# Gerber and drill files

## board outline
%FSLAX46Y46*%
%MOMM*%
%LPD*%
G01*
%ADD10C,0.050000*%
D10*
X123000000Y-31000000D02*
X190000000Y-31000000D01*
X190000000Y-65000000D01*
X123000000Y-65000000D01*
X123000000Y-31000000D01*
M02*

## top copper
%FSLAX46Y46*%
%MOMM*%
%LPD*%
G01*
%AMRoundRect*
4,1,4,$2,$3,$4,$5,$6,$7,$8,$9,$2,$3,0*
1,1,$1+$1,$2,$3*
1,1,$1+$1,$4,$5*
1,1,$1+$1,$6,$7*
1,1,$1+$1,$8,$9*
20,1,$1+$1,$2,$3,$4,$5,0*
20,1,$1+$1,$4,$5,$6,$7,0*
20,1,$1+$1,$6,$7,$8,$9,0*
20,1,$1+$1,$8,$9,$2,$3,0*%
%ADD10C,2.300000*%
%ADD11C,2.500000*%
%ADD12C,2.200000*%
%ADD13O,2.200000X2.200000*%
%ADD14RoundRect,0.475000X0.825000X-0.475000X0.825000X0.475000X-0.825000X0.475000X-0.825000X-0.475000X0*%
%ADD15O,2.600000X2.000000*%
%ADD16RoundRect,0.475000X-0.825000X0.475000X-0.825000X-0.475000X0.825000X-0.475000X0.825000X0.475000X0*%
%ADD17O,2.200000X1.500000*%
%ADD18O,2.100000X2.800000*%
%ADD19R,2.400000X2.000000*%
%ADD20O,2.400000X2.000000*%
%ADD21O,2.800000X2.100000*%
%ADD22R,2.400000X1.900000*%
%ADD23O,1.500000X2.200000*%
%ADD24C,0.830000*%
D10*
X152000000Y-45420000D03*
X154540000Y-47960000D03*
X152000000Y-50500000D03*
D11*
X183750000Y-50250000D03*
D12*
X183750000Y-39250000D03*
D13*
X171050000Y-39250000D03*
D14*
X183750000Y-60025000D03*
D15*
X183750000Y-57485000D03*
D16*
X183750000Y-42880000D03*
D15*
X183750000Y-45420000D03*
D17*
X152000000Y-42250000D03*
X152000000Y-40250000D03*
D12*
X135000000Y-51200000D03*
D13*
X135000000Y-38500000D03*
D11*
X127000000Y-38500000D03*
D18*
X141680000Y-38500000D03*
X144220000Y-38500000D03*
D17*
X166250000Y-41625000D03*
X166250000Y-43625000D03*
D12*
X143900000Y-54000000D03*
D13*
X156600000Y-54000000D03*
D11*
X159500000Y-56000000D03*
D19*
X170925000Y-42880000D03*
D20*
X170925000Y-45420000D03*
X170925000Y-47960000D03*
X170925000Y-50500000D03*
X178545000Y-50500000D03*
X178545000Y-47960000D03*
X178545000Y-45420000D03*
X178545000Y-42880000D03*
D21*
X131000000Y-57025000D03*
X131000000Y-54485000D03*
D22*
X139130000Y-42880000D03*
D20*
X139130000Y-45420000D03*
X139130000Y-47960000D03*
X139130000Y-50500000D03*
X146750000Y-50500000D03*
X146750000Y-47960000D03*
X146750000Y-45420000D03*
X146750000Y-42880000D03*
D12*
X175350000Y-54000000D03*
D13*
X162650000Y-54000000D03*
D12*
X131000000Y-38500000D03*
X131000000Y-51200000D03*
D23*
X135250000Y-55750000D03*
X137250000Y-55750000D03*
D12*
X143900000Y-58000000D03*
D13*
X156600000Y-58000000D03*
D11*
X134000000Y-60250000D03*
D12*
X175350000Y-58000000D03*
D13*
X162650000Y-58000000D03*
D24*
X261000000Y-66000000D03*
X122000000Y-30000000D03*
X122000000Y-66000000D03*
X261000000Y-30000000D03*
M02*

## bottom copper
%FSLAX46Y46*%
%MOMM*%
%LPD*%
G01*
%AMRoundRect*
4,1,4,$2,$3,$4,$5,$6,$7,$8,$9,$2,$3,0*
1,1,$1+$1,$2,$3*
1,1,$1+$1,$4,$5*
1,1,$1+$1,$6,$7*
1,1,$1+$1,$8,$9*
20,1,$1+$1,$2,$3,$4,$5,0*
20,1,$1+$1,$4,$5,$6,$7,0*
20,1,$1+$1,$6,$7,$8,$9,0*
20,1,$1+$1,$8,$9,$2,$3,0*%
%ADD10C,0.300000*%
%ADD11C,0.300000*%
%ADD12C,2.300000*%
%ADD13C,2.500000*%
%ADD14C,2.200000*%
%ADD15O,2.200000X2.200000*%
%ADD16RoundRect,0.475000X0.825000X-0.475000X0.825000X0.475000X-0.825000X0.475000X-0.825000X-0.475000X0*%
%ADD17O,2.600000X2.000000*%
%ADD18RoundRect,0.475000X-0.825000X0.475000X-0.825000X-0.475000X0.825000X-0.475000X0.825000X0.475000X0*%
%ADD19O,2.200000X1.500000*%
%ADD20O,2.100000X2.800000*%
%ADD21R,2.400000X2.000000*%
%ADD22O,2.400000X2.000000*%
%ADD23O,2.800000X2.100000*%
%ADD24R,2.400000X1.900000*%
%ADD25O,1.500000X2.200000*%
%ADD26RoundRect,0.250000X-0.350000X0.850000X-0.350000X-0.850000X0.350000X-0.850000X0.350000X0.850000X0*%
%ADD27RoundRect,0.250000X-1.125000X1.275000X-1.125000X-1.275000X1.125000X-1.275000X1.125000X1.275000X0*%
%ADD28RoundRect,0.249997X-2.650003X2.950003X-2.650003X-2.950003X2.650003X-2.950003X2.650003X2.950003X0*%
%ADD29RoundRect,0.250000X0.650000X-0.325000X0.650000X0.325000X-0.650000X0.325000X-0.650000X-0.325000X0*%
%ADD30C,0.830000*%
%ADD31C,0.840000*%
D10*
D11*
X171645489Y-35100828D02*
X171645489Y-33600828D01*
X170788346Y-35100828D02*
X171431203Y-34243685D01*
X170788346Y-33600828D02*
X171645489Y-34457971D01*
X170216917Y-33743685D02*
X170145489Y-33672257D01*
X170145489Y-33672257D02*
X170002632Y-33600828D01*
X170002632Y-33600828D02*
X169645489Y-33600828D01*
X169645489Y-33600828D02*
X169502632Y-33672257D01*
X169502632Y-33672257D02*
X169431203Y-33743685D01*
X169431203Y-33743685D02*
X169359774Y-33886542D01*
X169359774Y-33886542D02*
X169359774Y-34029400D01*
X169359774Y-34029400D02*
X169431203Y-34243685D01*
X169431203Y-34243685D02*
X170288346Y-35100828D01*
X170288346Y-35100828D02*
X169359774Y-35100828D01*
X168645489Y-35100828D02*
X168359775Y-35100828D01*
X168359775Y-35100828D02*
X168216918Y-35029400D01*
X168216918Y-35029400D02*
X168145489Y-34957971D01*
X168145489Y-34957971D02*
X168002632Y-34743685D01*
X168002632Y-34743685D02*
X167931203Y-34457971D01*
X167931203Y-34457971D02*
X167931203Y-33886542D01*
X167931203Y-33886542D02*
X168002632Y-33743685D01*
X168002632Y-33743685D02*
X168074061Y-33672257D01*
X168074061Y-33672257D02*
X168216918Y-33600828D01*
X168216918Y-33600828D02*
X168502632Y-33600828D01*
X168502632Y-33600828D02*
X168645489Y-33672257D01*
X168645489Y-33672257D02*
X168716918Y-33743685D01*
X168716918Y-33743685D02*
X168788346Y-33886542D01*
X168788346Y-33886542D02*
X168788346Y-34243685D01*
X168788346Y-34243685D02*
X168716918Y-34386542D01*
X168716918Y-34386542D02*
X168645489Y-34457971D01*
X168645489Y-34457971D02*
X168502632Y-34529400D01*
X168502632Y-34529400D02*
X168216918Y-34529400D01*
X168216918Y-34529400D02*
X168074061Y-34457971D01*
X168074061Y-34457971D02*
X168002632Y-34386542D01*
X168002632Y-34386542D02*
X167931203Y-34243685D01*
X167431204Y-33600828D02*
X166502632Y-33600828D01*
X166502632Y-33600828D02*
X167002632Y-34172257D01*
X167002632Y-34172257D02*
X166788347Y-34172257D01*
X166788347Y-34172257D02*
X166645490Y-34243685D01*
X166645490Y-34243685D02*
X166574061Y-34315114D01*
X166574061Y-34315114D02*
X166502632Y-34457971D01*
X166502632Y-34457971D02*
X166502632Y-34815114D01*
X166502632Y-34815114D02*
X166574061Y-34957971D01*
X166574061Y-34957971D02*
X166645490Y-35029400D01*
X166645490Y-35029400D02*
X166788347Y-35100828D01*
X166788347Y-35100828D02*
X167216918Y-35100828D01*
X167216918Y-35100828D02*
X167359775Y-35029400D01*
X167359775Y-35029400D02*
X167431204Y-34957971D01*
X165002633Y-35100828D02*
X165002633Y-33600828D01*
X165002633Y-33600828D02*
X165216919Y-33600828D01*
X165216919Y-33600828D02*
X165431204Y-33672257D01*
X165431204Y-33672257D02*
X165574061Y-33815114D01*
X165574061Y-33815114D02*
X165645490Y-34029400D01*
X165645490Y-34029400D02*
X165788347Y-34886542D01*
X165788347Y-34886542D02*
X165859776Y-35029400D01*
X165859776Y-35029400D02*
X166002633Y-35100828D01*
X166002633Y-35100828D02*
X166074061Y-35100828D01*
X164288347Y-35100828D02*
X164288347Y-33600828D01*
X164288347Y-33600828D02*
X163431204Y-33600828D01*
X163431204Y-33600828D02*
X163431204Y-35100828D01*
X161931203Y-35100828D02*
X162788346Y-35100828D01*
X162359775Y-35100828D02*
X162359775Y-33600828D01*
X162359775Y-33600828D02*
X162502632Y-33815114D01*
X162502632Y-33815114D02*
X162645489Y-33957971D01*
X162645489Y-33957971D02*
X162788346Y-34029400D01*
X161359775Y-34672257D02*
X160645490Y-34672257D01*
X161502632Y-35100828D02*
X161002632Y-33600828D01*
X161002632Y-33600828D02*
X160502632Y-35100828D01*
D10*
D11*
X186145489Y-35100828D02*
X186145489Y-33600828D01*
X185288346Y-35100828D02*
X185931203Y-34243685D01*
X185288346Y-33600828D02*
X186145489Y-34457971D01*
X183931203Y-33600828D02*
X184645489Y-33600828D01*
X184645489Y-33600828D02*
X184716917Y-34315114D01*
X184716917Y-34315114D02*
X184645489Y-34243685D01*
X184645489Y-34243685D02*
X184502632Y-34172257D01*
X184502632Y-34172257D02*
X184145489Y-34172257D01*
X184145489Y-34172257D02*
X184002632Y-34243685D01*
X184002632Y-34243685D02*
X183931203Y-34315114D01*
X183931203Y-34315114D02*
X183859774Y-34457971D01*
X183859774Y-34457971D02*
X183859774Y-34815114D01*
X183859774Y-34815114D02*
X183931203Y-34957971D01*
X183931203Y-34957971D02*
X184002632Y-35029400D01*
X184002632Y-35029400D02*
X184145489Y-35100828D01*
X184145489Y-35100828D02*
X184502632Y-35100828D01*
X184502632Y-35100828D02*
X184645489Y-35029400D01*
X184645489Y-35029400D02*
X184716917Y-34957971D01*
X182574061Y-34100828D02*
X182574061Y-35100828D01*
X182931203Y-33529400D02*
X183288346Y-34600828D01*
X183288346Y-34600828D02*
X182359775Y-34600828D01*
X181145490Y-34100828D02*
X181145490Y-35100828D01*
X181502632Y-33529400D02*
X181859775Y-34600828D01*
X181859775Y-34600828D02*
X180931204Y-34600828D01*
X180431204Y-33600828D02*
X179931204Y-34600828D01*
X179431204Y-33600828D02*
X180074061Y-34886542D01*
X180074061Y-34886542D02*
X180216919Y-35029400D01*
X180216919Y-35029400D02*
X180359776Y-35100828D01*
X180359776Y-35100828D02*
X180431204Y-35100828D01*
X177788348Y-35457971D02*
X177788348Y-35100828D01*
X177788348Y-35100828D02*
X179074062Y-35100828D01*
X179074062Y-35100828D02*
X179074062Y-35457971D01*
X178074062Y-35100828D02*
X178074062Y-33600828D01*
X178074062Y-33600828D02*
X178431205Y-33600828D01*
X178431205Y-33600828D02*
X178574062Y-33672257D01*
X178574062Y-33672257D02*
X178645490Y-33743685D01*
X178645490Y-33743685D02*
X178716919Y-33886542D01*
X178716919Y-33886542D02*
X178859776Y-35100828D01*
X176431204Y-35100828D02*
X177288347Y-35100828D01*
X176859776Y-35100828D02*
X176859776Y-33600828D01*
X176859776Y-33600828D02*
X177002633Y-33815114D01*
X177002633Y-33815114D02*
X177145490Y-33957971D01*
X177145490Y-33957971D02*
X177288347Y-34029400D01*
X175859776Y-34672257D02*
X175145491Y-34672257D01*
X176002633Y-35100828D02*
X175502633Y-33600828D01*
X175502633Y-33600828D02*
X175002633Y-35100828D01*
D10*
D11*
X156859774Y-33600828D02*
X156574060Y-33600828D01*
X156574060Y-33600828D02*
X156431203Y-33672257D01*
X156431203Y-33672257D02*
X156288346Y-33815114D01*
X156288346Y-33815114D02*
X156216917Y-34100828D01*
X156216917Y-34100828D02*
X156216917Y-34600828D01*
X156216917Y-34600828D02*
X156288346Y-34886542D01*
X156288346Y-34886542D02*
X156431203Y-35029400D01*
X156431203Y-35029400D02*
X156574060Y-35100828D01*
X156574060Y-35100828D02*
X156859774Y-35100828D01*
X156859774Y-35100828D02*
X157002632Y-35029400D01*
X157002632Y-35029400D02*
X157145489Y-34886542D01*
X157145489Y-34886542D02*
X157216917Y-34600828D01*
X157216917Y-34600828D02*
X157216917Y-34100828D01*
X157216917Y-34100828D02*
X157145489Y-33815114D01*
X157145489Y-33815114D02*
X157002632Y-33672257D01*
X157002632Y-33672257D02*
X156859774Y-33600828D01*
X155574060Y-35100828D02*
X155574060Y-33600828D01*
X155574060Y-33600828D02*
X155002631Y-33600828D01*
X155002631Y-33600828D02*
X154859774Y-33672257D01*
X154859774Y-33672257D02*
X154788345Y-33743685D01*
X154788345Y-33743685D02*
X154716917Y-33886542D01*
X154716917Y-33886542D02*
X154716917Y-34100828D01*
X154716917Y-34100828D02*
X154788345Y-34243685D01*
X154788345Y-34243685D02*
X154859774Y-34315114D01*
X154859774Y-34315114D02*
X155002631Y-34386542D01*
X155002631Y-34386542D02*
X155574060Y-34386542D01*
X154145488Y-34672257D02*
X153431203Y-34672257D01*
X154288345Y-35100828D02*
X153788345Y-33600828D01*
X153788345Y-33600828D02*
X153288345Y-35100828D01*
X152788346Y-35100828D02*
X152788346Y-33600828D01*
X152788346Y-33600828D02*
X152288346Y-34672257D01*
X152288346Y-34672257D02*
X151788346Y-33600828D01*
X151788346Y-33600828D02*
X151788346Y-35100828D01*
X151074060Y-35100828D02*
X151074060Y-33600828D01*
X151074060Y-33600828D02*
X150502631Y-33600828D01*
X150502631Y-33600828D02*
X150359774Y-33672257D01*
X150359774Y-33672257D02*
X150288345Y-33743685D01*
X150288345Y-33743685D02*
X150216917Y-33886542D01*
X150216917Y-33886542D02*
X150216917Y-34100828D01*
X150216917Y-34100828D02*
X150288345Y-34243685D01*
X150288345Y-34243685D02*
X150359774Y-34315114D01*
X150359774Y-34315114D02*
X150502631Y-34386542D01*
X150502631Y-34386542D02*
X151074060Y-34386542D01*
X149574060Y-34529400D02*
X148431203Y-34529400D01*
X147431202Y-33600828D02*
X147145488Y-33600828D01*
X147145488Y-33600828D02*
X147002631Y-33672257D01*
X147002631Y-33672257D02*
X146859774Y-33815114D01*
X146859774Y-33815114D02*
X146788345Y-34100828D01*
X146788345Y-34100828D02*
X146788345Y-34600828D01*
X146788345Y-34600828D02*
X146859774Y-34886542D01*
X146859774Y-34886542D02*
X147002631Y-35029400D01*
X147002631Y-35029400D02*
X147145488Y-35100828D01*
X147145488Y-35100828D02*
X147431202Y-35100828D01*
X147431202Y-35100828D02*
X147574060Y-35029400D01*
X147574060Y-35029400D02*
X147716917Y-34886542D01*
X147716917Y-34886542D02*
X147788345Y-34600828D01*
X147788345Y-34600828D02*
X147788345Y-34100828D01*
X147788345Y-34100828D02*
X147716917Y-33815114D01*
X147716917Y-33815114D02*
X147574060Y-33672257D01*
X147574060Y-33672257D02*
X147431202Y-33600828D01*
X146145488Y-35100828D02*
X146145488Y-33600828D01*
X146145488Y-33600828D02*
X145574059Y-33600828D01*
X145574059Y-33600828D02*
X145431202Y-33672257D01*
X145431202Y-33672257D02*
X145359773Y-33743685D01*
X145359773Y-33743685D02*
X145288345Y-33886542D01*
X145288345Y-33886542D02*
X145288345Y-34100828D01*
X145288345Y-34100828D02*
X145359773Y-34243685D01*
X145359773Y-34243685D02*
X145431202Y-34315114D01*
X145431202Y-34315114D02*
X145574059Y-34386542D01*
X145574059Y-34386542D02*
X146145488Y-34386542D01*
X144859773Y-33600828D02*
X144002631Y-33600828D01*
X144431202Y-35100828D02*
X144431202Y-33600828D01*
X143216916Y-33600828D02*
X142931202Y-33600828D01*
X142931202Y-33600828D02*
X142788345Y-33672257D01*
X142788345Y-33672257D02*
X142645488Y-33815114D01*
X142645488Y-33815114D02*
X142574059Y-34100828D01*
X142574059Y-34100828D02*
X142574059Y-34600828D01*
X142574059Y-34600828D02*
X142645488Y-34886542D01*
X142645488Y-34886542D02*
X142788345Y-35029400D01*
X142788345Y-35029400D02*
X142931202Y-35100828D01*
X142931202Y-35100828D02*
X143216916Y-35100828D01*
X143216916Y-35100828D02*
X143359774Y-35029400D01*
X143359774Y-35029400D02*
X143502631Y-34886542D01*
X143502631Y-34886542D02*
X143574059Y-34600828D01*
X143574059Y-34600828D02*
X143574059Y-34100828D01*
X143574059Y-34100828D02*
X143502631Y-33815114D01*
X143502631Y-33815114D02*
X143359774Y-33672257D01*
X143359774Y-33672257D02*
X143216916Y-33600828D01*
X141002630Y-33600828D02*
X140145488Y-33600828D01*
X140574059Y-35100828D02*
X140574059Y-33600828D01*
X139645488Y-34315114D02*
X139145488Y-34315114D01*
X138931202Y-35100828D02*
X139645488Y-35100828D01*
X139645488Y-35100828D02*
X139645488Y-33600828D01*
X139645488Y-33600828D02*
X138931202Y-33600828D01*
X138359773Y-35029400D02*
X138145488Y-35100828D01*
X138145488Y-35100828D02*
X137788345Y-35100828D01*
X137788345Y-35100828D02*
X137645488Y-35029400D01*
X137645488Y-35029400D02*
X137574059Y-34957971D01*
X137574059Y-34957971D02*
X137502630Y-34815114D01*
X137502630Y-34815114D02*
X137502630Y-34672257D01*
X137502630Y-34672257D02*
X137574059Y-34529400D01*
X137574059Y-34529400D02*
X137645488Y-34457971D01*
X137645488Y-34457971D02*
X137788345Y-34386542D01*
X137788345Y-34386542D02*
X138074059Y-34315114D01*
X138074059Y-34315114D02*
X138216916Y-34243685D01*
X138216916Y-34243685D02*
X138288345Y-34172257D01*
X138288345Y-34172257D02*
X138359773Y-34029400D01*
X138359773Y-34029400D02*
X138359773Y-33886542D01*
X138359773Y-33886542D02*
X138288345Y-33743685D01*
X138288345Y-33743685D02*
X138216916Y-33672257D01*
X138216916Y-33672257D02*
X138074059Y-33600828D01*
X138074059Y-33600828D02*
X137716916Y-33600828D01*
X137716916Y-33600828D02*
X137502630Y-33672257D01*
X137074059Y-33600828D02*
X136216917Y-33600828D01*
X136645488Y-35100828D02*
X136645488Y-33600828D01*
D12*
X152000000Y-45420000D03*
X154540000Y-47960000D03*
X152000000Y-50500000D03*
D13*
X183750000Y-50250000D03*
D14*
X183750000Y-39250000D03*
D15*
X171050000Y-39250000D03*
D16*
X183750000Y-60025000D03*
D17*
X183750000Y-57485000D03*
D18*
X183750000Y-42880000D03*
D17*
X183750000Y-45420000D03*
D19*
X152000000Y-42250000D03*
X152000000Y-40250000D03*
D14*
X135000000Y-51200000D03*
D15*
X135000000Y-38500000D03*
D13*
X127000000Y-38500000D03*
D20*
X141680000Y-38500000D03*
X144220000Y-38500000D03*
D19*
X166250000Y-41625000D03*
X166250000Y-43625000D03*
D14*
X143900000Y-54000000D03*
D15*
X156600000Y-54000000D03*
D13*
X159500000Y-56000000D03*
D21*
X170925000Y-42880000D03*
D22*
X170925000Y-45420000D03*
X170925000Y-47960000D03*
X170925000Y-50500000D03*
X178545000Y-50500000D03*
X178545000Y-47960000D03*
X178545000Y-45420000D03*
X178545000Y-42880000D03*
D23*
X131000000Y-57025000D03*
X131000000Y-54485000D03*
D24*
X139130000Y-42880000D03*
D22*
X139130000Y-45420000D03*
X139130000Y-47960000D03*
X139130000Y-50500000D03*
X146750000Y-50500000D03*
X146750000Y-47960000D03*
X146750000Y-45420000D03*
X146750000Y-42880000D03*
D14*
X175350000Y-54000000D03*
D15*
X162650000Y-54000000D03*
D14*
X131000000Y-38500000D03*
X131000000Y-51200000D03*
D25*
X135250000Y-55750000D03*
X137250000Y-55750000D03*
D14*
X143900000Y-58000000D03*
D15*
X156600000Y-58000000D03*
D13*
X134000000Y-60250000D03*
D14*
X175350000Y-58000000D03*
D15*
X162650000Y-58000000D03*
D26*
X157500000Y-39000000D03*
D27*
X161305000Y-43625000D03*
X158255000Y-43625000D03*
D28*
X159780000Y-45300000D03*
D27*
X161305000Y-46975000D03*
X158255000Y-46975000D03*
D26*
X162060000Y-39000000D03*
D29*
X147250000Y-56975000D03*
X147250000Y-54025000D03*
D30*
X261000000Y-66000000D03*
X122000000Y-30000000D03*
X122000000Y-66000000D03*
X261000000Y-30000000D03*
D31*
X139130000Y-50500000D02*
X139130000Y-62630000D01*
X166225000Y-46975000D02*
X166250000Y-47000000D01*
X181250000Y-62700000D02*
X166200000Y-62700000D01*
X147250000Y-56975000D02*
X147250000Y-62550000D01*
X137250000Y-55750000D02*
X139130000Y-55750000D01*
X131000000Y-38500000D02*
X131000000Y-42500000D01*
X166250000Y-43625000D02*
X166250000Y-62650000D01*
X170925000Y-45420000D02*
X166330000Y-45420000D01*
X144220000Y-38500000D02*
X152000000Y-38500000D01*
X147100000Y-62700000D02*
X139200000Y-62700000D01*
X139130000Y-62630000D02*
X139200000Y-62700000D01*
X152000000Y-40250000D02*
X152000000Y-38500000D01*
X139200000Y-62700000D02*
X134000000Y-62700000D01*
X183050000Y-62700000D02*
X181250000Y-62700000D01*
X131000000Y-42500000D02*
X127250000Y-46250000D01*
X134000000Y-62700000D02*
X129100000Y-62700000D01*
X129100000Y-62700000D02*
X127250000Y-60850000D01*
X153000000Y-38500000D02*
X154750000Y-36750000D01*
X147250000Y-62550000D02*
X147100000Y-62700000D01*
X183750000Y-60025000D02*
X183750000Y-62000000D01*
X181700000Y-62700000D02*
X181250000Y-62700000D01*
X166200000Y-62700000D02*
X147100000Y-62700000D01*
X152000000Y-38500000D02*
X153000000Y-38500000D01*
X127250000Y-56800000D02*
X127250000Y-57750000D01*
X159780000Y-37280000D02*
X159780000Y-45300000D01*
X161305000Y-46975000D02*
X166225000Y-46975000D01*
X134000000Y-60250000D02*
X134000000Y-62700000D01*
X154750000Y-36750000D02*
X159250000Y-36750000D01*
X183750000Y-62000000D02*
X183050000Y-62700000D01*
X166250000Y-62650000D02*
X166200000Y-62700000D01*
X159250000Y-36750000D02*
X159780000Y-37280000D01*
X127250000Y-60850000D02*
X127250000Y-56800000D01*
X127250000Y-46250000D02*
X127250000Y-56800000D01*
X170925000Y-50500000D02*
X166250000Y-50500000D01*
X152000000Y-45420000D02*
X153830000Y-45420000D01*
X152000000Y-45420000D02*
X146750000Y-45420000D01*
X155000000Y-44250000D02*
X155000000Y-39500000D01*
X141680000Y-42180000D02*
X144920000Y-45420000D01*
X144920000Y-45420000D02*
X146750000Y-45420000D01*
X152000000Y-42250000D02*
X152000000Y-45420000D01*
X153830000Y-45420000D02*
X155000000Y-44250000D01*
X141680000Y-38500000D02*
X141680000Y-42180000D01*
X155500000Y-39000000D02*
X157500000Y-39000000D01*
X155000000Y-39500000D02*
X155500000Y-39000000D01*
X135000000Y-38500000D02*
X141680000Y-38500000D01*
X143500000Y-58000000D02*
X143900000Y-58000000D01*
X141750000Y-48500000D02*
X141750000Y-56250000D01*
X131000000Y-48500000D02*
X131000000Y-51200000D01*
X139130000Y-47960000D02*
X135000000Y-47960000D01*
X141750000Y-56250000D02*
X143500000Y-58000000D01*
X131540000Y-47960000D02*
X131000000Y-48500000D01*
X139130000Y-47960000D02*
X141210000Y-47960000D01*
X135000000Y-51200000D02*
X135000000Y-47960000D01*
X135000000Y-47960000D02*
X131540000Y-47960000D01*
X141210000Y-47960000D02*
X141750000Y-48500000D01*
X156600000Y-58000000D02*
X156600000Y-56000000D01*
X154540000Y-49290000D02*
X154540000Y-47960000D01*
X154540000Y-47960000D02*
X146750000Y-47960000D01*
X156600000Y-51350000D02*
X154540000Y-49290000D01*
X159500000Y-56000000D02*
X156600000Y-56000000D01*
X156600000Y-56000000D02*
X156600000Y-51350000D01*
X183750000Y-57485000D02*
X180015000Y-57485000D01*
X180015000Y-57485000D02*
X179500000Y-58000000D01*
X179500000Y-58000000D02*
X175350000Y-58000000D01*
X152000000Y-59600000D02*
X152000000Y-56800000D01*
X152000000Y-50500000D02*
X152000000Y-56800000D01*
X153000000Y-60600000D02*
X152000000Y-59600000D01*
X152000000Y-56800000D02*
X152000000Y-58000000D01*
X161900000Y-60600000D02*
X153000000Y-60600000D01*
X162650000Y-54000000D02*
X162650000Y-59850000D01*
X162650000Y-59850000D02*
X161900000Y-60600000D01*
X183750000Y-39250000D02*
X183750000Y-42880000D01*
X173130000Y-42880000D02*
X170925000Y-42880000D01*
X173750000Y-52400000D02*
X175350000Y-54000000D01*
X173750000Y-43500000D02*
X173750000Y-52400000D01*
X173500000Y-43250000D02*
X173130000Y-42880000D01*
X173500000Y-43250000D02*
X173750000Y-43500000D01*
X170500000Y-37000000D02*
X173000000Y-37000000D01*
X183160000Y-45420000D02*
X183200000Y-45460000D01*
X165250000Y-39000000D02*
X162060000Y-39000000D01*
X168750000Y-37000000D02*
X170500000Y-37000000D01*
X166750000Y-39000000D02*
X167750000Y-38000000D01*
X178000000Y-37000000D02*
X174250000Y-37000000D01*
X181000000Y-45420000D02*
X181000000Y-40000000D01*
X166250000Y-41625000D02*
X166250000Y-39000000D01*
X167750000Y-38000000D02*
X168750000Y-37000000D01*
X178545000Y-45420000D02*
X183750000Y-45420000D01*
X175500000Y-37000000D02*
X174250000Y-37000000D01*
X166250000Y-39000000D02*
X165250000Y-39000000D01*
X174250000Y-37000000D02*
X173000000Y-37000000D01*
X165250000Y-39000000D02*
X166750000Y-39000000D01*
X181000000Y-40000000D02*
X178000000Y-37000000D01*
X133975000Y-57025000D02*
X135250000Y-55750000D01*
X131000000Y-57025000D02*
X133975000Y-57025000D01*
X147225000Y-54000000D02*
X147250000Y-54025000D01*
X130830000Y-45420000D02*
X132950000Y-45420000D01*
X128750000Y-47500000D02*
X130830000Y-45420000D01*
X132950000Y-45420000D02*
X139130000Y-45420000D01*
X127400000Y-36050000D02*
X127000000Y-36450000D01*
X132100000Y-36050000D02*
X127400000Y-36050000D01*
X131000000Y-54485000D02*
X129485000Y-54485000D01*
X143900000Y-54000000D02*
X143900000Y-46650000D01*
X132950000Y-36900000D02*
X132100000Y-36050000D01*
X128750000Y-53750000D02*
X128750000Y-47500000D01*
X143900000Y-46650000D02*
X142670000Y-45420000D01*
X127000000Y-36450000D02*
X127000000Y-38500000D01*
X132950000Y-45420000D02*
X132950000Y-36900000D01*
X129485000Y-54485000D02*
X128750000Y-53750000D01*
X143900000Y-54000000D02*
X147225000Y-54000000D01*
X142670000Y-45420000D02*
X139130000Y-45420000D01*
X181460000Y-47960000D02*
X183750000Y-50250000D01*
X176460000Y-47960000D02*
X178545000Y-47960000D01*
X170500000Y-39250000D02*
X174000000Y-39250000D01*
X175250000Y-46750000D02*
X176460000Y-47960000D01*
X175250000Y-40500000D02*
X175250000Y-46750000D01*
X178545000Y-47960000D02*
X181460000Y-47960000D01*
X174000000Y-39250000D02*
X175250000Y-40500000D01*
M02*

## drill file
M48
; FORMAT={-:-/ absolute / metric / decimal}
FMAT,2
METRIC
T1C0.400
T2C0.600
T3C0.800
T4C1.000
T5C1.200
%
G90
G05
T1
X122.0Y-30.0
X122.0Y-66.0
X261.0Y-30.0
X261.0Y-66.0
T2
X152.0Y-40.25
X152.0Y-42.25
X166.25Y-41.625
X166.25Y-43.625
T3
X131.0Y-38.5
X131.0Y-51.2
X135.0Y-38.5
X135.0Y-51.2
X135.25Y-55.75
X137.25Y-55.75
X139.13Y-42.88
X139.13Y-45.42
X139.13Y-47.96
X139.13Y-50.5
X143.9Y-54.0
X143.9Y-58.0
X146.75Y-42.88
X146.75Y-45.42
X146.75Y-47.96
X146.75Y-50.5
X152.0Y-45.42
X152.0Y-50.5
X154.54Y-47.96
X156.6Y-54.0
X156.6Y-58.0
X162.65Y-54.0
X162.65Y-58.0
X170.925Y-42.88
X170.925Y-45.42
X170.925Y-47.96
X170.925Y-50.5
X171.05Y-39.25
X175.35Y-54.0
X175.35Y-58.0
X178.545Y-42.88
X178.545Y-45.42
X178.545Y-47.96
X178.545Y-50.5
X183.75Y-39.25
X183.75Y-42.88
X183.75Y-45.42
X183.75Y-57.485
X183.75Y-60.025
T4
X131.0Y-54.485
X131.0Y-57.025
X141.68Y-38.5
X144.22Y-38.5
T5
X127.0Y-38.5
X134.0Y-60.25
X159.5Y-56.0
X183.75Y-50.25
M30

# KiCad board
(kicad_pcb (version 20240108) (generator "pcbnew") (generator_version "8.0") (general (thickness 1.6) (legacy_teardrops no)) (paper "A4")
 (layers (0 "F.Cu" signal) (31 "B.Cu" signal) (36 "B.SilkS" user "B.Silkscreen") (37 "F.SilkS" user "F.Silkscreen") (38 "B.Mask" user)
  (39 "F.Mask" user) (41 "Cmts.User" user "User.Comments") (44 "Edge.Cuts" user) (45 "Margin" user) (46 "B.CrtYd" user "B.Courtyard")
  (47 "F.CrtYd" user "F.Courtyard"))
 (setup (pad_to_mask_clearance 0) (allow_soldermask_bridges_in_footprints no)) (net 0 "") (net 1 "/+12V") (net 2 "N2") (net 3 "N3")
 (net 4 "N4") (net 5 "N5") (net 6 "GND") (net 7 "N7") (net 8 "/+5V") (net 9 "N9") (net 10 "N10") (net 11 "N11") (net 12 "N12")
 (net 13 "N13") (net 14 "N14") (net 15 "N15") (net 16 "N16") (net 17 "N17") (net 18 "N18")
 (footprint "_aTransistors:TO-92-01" (layer "F.Cu") (at 152 47.953903 -90)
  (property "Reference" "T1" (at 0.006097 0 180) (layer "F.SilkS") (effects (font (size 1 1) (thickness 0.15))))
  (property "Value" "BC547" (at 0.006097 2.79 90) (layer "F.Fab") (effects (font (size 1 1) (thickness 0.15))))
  (pad "1" thru_hole circle (at -2.533903 0 270) (size 2.3 2.3) (drill 0.8) (layers "*.Cu" "*.Mask") (remove_unused_layers no)
   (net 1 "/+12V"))
  (pad "2" thru_hole circle (at 0.006097 -2.54 270) (size 2.3 2.3) (drill 0.8) (layers "*.Cu" "*.Mask") (remove_unused_layers no)
   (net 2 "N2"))
  (pad "3" thru_hole circle (at 2.546097 0 270) (size 2.3 2.3) (drill 0.8) (layers "*.Cu" "*.Mask") (remove_unused_layers no) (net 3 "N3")))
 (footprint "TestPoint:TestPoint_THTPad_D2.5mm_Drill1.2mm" (layer "F.Cu") (at 183.75 50.25)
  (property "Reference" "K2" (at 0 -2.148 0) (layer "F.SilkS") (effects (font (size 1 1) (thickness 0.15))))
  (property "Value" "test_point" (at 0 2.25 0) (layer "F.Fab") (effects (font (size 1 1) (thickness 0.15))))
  (pad "1" thru_hole circle (at 0 0) (size 2.5 2.5) (drill 1.2) (layers "*.Cu" "*.Mask") (remove_unused_layers no) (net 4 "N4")))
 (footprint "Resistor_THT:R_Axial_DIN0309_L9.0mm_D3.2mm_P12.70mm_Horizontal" (layer "F.Cu") (at 183.75 39.25 180)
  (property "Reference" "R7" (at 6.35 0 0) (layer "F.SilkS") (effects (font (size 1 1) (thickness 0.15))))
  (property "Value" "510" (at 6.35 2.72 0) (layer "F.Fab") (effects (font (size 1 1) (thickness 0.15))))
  (pad "1" thru_hole circle (at 0 0 180) (size 2.2 2.2) (drill 0.8) (layers "*.Cu" "*.Mask") (remove_unused_layers no) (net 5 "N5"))
  (pad "2" thru_hole oval (at 12.7 0 180) (size 2.2 2.2) (drill 0.8) (layers "*.Cu" "*.Mask") (remove_unused_layers no) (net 4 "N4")))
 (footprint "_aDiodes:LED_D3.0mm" (layer "F.Cu") (at 183.75 60.025 90)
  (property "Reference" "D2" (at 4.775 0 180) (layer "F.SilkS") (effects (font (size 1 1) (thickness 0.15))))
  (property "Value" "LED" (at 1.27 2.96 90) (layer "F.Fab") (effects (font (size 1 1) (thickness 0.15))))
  (pad "1" thru_hole roundrect (at 0 0 90) (size 1.9 2.6) (drill 0.8) (layers "*.Cu" "*.Mask") (remove_unused_layers no)
   (roundrect_rratio 0.25) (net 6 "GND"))
  (pad "2" thru_hole oval (at 2.54 0 90) (size 2 2.6) (drill 0.8) (layers "*.Cu" "*.Mask") (remove_unused_layers no) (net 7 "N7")))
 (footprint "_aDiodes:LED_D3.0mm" (layer "F.Cu") (at 183.75 42.88 -90)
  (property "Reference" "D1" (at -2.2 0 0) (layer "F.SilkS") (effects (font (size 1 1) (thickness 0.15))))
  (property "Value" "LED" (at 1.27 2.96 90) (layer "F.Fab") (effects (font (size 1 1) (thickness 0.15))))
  (pad "1" thru_hole roundrect (at 0 0 270) (size 1.9 2.6) (drill 0.8) (layers "*.Cu" "*.Mask") (remove_unused_layers no)
   (roundrect_rratio 0.25) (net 5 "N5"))
  (pad "2" thru_hole oval (at 2.54 0 270) (size 2 2.6) (drill 0.8) (layers "*.Cu" "*.Mask") (remove_unused_layers no) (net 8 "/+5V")))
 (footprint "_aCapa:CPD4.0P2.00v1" (layer "F.Cu") (at 152 41.25 90)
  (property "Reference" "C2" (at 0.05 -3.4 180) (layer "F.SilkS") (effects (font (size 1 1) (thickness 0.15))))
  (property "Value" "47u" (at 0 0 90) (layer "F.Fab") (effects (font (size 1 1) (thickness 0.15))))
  (pad "1" thru_hole oval (at -1 0 90) (size 1.5 2.2) (drill 0.6) (layers "*.Cu" "*.Mask") (remove_unused_layers no) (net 1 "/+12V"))
  (pad "2" thru_hole oval (at 1 0 90) (size 1.5 2.2) (drill 0.6) (layers "*.Cu" "*.Mask") (remove_unused_layers no) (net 6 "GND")))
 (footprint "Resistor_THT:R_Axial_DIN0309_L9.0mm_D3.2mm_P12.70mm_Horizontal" (layer "F.Cu") (at 135 51.2 90)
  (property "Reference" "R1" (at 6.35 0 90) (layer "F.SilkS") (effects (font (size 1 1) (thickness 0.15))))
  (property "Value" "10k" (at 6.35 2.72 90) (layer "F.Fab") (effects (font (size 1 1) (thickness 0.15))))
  (pad "1" thru_hole circle (at 0 0 90) (size 2.2 2.2) (drill 0.8) (layers "*.Cu" "*.Mask") (remove_unused_layers no) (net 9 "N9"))
  (pad "2" thru_hole oval (at 12.7 0 90) (size 2.2 2.2) (drill 0.8) (layers "*.Cu" "*.Mask") (remove_unused_layers no) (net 1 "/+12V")))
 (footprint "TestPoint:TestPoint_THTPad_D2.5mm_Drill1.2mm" (layer "F.Cu") (at 127 38.5)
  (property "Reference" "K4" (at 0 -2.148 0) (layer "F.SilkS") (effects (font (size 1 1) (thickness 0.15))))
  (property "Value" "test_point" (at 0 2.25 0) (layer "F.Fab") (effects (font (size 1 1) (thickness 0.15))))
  (pad "1" thru_hole circle (at 0 0) (size 2.5 2.5) (drill 1.2) (layers "*.Cu" "*.Mask") (remove_unused_layers no) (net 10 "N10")))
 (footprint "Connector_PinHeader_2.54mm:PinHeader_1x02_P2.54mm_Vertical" (layer "F.Cu") (at 141.68 38.5 90)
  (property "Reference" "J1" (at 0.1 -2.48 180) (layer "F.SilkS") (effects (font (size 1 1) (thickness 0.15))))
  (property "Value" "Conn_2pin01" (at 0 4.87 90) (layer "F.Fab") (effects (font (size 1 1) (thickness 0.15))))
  (pad "1" thru_hole oval (at 0 0 90) (size 2.8 2.1) (drill 1) (layers "*.Cu" "*.Mask") (remove_unused_layers no) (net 1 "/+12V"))
  (pad "2" thru_hole oval (at 0 2.54 90) (size 2.8 2.1) (drill 1) (layers "*.Cu" "*.Mask") (remove_unused_layers no) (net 6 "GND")))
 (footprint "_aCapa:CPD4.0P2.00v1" (layer "F.Cu") (at 166.25 42.625 -90)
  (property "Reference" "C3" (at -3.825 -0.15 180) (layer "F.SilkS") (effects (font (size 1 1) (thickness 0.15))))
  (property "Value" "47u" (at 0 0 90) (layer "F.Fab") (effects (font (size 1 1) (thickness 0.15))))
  (pad "1" thru_hole oval (at -1 0 270) (size 1.5 2.2) (drill 0.6) (layers "*.Cu" "*.Mask") (remove_unused_layers no) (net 8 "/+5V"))
  (pad "2" thru_hole oval (at 1 0 270) (size 1.5 2.2) (drill 0.6) (layers "*.Cu" "*.Mask") (remove_unused_layers no) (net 6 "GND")))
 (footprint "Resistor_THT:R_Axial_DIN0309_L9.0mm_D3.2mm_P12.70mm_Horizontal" (layer "F.Cu") (at 143.9 54)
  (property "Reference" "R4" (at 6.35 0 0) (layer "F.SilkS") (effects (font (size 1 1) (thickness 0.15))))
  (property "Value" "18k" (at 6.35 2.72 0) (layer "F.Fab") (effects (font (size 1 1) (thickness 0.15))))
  (pad "1" thru_hole circle (at 0 0) (size 2.2 2.2) (drill 0.8) (layers "*.Cu" "*.Mask") (remove_unused_layers no) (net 10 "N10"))
  (pad "2" thru_hole oval (at 12.7 0) (size 2.2 2.2) (drill 0.8) (layers "*.Cu" "*.Mask") (remove_unused_layers no) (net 2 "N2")))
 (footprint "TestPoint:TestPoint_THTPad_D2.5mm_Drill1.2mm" (layer "F.Cu") (at 159.5 56)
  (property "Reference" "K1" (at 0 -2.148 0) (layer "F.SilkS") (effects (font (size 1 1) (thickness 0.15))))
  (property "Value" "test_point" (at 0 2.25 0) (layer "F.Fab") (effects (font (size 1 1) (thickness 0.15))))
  (pad "1" thru_hole circle (at 0 0) (size 2.5 2.5) (drill 1.2) (layers "*.Cu" "*.Mask") (remove_unused_layers no) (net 2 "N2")))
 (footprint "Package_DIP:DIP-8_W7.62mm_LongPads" (layer "F.Cu") (at 170.925 42.88)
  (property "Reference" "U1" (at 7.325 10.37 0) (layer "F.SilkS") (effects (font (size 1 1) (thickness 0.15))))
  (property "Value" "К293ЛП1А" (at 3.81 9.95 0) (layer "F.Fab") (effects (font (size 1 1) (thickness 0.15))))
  (pad "1" thru_hole rect (at 0 0) (size 2.4 2) (drill 0.8) (layers "*.Cu" "*.Mask") (remove_unused_layers no) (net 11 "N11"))
  (pad "2" thru_hole oval (at 0 2.54) (size 2.4 2) (drill 0.8) (layers "*.Cu" "*.Mask") (remove_unused_layers no) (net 6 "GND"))
  (pad "3" thru_hole oval (at 0 5.08) (size 2.4 2) (drill 0.8) (layers "*.Cu" "*.Mask") (remove_unused_layers no) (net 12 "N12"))
  (pad "4" thru_hole oval (at 0 7.62) (size 2.4 2) (drill 0.8) (layers "*.Cu" "*.Mask") (remove_unused_layers no) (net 6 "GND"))
  (pad "5" thru_hole oval (at 7.62 7.62) (size 2.4 2) (drill 0.8) (layers "*.Cu" "*.Mask") (remove_unused_layers no) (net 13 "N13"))
  (pad "6" thru_hole oval (at 7.62 5.08) (size 2.4 2) (drill 0.8) (layers "*.Cu" "*.Mask") (remove_unused_layers no) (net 4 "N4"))
  (pad "7" thru_hole oval (at 7.62 2.54) (size 2.4 2) (drill 0.8) (layers "*.Cu" "*.Mask") (remove_unused_layers no) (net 8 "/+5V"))
  (pad "8" thru_hole oval (at 7.62 0) (size 2.4 2) (drill 0.8) (layers "*.Cu" "*.Mask") (remove_unused_layers no) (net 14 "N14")))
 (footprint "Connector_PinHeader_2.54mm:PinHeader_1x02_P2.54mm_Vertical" (layer "F.Cu") (at 131 57.025 180)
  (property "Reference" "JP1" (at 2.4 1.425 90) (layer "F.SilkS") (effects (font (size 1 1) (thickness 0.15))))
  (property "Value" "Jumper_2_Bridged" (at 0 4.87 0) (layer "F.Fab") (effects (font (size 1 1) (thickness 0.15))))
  (pad "1" thru_hole oval (at 0 0 180) (size 2.8 2.1) (drill 1) (layers "*.Cu" "*.Mask") (remove_unused_layers no) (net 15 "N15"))
  (pad "2" thru_hole oval (at 0 2.54 180) (size 2.8 2.1) (drill 1) (layers "*.Cu" "*.Mask") (remove_unused_layers no) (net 10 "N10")))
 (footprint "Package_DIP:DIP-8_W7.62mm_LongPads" (layer "F.Cu") (at 139.13 42.88)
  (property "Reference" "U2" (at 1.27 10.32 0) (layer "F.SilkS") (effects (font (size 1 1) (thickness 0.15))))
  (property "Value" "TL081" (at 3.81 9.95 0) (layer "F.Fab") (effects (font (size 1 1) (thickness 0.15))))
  (pad "1" thru_hole rect (at 0 0) (size 2.4 1.9) (drill 0.8) (layers "*.Cu" "*.Mask") (remove_unused_layers no) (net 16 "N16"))
  (pad "2" thru_hole oval (at 0 2.54) (size 2.4 2) (drill 0.8) (layers "*.Cu" "*.Mask") (remove_unused_layers no) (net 10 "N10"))
  (pad "3" thru_hole oval (at 0 5.08) (size 2.4 2) (drill 0.8) (layers "*.Cu" "*.Mask") (remove_unused_layers no) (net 9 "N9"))
  (pad "4" thru_hole oval (at 0 7.62) (size 2.4 2) (drill 0.8) (layers "*.Cu" "*.Mask") (remove_unused_layers no) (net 6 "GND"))
  (pad "5" thru_hole oval (at 7.62 7.62) (size 2.4 2) (drill 0.8) (layers "*.Cu" "*.Mask") (remove_unused_layers no) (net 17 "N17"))
  (pad "6" thru_hole oval (at 7.62 5.08) (size 2.4 2) (drill 0.8) (layers "*.Cu" "*.Mask") (remove_unused_layers no) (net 2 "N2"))
  (pad "7" thru_hole oval (at 7.62 2.54) (size 2.4 2) (drill 0.8) (layers "*.Cu" "*.Mask") (remove_unused_layers no) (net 1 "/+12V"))
  (pad "8" thru_hole oval (at 7.62 0) (size 2.4 2) (drill 0.8) (layers "*.Cu" "*.Mask") (remove_unused_layers no) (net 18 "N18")))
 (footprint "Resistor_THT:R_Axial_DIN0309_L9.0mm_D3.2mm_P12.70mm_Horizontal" (layer "F.Cu") (at 175.35 54 180)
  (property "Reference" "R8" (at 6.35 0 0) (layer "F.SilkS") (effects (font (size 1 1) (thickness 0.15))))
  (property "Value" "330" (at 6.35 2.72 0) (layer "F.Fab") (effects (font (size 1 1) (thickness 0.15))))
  (pad "1" thru_hole circle (at 0 0 180) (size 2.2 2.2) (drill 0.8) (layers "*.Cu" "*.Mask") (remove_unused_layers no) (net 11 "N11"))
  (pad "2" thru_hole oval (at 12.7 0 180) (size 2.2 2.2) (drill 0.8) (layers "*.Cu" "*.Mask") (remove_unused_layers no) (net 3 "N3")))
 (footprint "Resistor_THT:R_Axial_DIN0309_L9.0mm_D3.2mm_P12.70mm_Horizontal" (layer "F.Cu") (at 131 38.5 -90)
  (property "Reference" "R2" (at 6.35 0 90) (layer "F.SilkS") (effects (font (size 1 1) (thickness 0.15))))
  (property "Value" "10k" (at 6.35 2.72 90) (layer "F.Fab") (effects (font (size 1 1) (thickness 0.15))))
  (pad "1" thru_hole circle (at 0 0 270) (size 2.2 2.2) (drill 0.8) (layers "*.Cu" "*.Mask") (remove_unused_layers no) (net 6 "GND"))
  (pad "2" thru_hole circle (at 12.7 0 270) (size 2.2 2.2) (drill 0.8) (layers "*.Cu" "*.Mask") (remove_unused_layers no) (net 9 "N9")))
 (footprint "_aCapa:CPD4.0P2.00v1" (layer "F.Cu") (at 136.25 55.75)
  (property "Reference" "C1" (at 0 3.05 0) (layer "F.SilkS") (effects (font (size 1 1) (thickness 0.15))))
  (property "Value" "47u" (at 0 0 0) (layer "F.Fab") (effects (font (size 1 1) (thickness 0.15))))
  (pad "1" thru_hole oval (at -1 0) (size 1.5 2.2) (drill 0.8) (layers "*.Cu" "*.Mask") (remove_unused_layers no) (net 15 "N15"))
  (pad "2" thru_hole oval (at 1 0) (size 1.5 2.2) (drill 0.8) (layers "*.Cu" "*.Mask") (remove_unused_layers no) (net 6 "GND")))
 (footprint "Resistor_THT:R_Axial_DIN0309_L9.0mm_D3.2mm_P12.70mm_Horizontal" (layer "F.Cu") (at 143.9 58)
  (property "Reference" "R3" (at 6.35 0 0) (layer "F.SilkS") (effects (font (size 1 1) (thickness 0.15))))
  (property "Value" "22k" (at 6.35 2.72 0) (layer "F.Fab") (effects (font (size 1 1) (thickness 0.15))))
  (pad "1" thru_hole circle (at 0 0) (size 2.2 2.2) (drill 0.8) (layers "*.Cu" "*.Mask") (remove_unused_layers no) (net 9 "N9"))
  (pad "2" thru_hole oval (at 12.7 0) (size 2.2 2.2) (drill 0.8) (layers "*.Cu" "*.Mask") (remove_unused_layers no) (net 2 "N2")))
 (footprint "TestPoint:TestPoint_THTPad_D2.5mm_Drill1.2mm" (layer "F.Cu") (at 134 60.25)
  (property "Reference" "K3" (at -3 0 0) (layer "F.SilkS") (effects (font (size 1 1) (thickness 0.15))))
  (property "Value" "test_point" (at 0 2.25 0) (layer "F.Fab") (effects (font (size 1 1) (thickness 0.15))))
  (pad "1" thru_hole circle (at 0 0) (size 2.5 2.5) (drill 1.2) (layers "*.Cu" "*.Mask") (remove_unused_layers no) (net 6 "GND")))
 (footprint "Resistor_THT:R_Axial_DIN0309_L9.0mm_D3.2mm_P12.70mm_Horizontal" (layer "F.Cu") (at 175.35 58 180)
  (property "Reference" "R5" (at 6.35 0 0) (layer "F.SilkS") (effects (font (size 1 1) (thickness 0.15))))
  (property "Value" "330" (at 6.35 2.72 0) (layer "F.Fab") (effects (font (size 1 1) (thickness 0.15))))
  (pad "1" thru_hole circle (at 0 0 180) (size 2.2 2.2) (drill 0.8) (layers "*.Cu" "*.Mask") (remove_unused_layers no) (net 7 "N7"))
  (pad "2" thru_hole oval (at 12.7 0 180) (size 2.2 2.2) (drill 0.8) (layers "*.Cu" "*.Mask") (remove_unused_layers no) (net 3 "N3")))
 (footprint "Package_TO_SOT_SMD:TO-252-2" (layer "B.Cu") (at 159.78 44.04 -90)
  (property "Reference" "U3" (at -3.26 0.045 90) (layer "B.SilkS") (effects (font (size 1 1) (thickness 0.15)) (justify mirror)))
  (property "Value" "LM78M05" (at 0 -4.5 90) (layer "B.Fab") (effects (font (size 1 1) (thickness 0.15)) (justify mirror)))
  (pad "1" smd roundrect (at -5.04 2.28 270) (size 2.2 1.2) (layers "B.Cu" "B.Paste" "B.Mask") (roundrect_rratio 0.208333) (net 1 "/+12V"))
  (pad "2" smd roundrect (at -0.415 -1.525 270) (size 3.05 2.75) (layers "B.Cu" "B.Paste") (roundrect_rratio 0.090909) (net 6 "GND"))
  (pad "2" smd roundrect (at -0.415 1.525 270) (size 3.05 2.75) (layers "B.Cu" "B.Paste") (roundrect_rratio 0.090909) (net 6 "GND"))
  (pad "2" smd roundrect (at 1.26 0 270) (size 6.4 5.8) (layers "B.Cu" "B.Mask") (roundrect_rratio 0.043103) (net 6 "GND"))
  (pad "2" smd roundrect (at 2.935 -1.525 270) (size 3.05 2.75) (layers "B.Cu" "B.Paste") (roundrect_rratio 0.090909) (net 6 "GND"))
  (pad "2" smd roundrect (at 2.935 1.525 270) (size 3.05 2.75) (layers "B.Cu" "B.Paste") (roundrect_rratio 0.090909) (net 6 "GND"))
  (pad "3" smd roundrect (at -5.04 -2.28 270) (size 2.2 1.2) (layers "B.Cu" "B.Paste" "B.Mask") (roundrect_rratio 0.208333) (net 8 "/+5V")))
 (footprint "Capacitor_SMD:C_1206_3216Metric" (layer "B.Cu") (at 147.25 55.5 90)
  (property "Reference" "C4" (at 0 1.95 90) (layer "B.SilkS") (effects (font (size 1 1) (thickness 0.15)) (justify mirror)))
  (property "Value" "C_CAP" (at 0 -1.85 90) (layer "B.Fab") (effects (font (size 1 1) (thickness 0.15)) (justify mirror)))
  (pad "1" smd roundrect (at -1.475 0 90) (size 1.15 1.8) (layers "B.Cu" "B.Paste" "B.Mask") (roundrect_rratio 0.217391) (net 6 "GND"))
  (pad "2" smd roundrect (at 1.475 0 90) (size 1.15 1.8) (layers "B.Cu" "B.Paste" "B.Mask") (roundrect_rratio 0.217391) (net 10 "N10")))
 (gr_rect (start 123 31) (end 190 65) (stroke (width 0.05) (type default)) (fill none) (layer "Edge.Cuts"))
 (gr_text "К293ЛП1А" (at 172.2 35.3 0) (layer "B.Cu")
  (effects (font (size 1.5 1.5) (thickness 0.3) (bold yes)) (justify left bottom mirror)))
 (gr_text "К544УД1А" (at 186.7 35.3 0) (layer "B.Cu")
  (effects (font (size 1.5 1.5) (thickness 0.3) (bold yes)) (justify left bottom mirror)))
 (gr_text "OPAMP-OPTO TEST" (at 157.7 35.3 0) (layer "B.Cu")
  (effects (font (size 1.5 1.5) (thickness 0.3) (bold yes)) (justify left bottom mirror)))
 (via (at 261 66) (size 0.83) (drill 0.4) (layers "F.Cu" "B.Cu") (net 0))
 (via (at 122 30) (size 0.83) (drill 0.4) (layers "F.Cu" "B.Cu") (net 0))
 (via (at 122 66) (size 0.83) (drill 0.4) (layers "F.Cu" "B.Cu") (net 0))
 (via (at 261 30) (size 0.83) (drill 0.4) (layers "F.Cu" "B.Cu") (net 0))
 (segment (start 139.13 50.5) (end 139.13 62.63) (width 0.84) (layer "B.Cu") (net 6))
 (segment (start 166.225 46.975) (end 166.25 47) (width 0.84) (layer "B.Cu") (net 6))
 (segment (start 181.25 62.7) (end 166.2 62.7) (width 0.84) (layer "B.Cu") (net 6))
 (segment (start 147.25 56.975) (end 147.25 62.55) (width 0.84) (layer "B.Cu") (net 6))
 (segment (start 137.25 55.75) (end 139.13 55.75) (width 0.84) (layer "B.Cu") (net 6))
 (segment (start 131 38.5) (end 131 42.5) (width 0.84) (layer "B.Cu") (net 6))
 (segment (start 166.25 43.625) (end 166.25 62.65) (width 0.84) (layer "B.Cu") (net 6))
 (segment (start 170.925 45.42) (end 166.33 45.42) (width 0.84) (layer "B.Cu") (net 6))
 (segment (start 144.22 38.5) (end 152 38.5) (width 0.84) (layer "B.Cu") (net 6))
 (segment (start 147.1 62.7) (end 139.2 62.7) (width 0.84) (layer "B.Cu") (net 6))
 (segment (start 139.13 62.63) (end 139.2 62.7) (width 0.84) (layer "B.Cu") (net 6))
 (segment (start 152 40.25) (end 152 38.5) (width 0.84) (layer "B.Cu") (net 6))
 (segment (start 139.2 62.7) (end 134 62.7) (width 0.84) (layer "B.Cu") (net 6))
 (segment (start 183.05 62.7) (end 181.25 62.7) (width 0.84) (layer "B.Cu") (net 6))
 (segment (start 131 42.5) (end 127.25 46.25) (width 0.84) (layer "B.Cu") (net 6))
 (segment (start 134 62.7) (end 129.1 62.7) (width 0.84) (layer "B.Cu") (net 6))
 (segment (start 129.1 62.7) (end 127.25 60.85) (width 0.84) (layer "B.Cu") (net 6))
 (segment (start 153 38.5) (end 154.75 36.75) (width 0.84) (layer "B.Cu") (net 6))
 (segment (start 147.25 62.55) (end 147.1 62.7) (width 0.84) (layer "B.Cu") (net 6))
 (segment (start 183.75 60.025) (end 183.75 62) (width 0.84) (layer "B.Cu") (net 6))
 (segment (start 181.7 62.7) (end 181.25 62.7) (width 0.84) (layer "B.Cu") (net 6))
 (segment (start 166.2 62.7) (end 147.1 62.7) (width 0.84) (layer "B.Cu") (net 6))
 (segment (start 152 38.5) (end 153 38.5) (width 0.84) (layer "B.Cu") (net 6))
 (segment (start 127.25 56.8) (end 127.25 57.75) (width 0.84) (layer "B.Cu") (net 6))
 (segment (start 159.78 37.28) (end 159.78 45.3) (width 0.84) (layer "B.Cu") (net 6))
 (segment (start 161.305 46.975) (end 166.225 46.975) (width 0.84) (layer "B.Cu") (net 6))
 (segment (start 134 60.25) (end 134 62.7) (width 0.84) (layer "B.Cu") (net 6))
 (segment (start 154.75 36.75) (end 159.25 36.75) (width 0.84) (layer "B.Cu") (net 6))
 (segment (start 183.75 62) (end 183.05 62.7) (width 0.84) (layer "B.Cu") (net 6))
 (segment (start 166.25 62.65) (end 166.2 62.7) (width 0.84) (layer "B.Cu") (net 6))
 (segment (start 159.25 36.75) (end 159.78 37.28) (width 0.84) (layer "B.Cu") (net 6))
 (segment (start 127.25 60.85) (end 127.25 56.8) (width 0.84) (layer "B.Cu") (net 6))
 (segment (start 127.25 46.25) (end 127.25 56.8) (width 0.84) (layer "B.Cu") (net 6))
 (segment (start 170.925 50.5) (end 166.25 50.5) (width 0.84) (layer "B.Cu") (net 6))
 (segment (start 152 45.42) (end 153.83 45.42) (width 0.84) (layer "B.Cu") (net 1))
 (segment (start 152 45.42) (end 146.75 45.42) (width 0.84) (layer "B.Cu") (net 1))
 (segment (start 155 44.25) (end 155 39.5) (width 0.84) (layer "B.Cu") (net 1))
 (segment (start 141.68 42.18) (end 144.92 45.42) (width 0.84) (layer "B.Cu") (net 1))
 (segment (start 144.92 45.42) (end 146.75 45.42) (width 0.84) (layer "B.Cu") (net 1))
 (segment (start 152 42.25) (end 152 45.42) (width 0.84) (layer "B.Cu") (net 1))
 (segment (start 153.83 45.42) (end 155 44.25) (width 0.84) (layer "B.Cu") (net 1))
 (segment (start 141.68 38.5) (end 141.68 42.18) (width 0.84) (layer "B.Cu") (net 1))
 (segment (start 155.5 39) (end 157.5 39) (width 0.84) (layer "B.Cu") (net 1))
 (segment (start 155 39.5) (end 155.5 39) (width 0.84) (layer "B.Cu") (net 1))
 (segment (start 135 38.5) (end 141.68 38.5) (width 0.84) (layer "B.Cu") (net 1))
 (segment (start 143.5 58) (end 143.9 58) (width 0.84) (layer "B.Cu") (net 9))
 (segment (start 141.75 48.5) (end 141.75 56.25) (width 0.84) (layer "B.Cu") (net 9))
 (segment (start 131 48.5) (end 131 51.2) (width 0.84) (layer "B.Cu") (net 9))
 (segment (start 139.13 47.96) (end 135 47.96) (width 0.84) (layer "B.Cu") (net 9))
 (segment (start 141.75 56.25) (end 143.5 58) (width 0.84) (layer "B.Cu") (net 9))
 (segment (start 131.54 47.96) (end 131 48.5) (width 0.84) (layer "B.Cu") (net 9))
 (segment (start 139.13 47.96) (end 141.21 47.96) (width 0.84) (layer "B.Cu") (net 9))
 (segment (start 135 51.2) (end 135 47.96) (width 0.84) (layer "B.Cu") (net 9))
 (segment (start 135 47.96) (end 131.54 47.96) (width 0.84) (layer "B.Cu") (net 9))
 (segment (start 141.21 47.96) (end 141.75 48.5) (width 0.84) (layer "B.Cu") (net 9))
 (segment (start 156.6 58) (end 156.6 56) (width 0.84) (layer "B.Cu") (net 2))
 (segment (start 154.54 49.29) (end 154.54 47.96) (width 0.84) (layer "B.Cu") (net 2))
 (segment (start 154.54 47.96) (end 146.75 47.96) (width 0.84) (layer "B.Cu") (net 2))
 (segment (start 156.6 51.35) (end 154.54 49.29) (width 0.84) (layer "B.Cu") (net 2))
 (segment (start 159.5 56) (end 156.6 56) (width 0.84) (layer "B.Cu") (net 2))
 (segment (start 156.6 56) (end 156.6 51.35) (width 0.84) (layer "B.Cu") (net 2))
 (segment (start 183.75 57.485) (end 180.015 57.485) (width 0.84) (layer "B.Cu") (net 7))
 (segment (start 180.015 57.485) (end 179.5 58) (width 0.84) (layer "B.Cu") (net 7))
 (segment (start 179.5 58) (end 175.35 58) (width 0.84) (layer "B.Cu") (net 7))
 (segment (start 152 59.6) (end 152 56.8) (width 0.84) (layer "B.Cu") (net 3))
 (segment (start 152 50.5) (end 152 56.8) (width 0.84) (layer "B.Cu") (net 3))
 (segment (start 153 60.6) (end 152 59.6) (width 0.84) (layer "B.Cu") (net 3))
 (segment (start 152 56.8) (end 152 58) (width 0.84) (layer "B.Cu") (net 3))
 (segment (start 161.9 60.6) (end 153 60.6) (width 0.84) (layer "B.Cu") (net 3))
 (segment (start 162.65 54) (end 162.65 59.85) (width 0.84) (layer "B.Cu") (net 3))
 (segment (start 162.65 59.85) (end 161.9 60.6) (width 0.84) (layer "B.Cu") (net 3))
 (segment (start 183.75 39.25) (end 183.75 42.88) (width 0.84) (layer "B.Cu") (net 5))
 (segment (start 173.13 42.88) (end 170.925 42.88) (width 0.84) (layer "B.Cu") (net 11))
 (segment (start 173.75 52.4) (end 175.35 54) (width 0.84) (layer "B.Cu") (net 11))
 (segment (start 173.75 43.5) (end 173.75 52.4) (width 0.84) (layer "B.Cu") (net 11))
 (segment (start 173.5 43.25) (end 173.13 42.88) (width 0.84) (layer "B.Cu") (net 11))
 (segment (start 173.5 43.25) (end 173.75 43.5) (width 0.84) (layer "B.Cu") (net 11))
 (segment (start 170.5 37) (end 173 37) (width 0.84) (layer "B.Cu") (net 8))
 (segment (start 183.16 45.42) (end 183.2 45.46) (width 0.84) (layer "B.Cu") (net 8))
 (segment (start 165.25 39) (end 162.06 39) (width 0.84) (layer "B.Cu") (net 8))
 (segment (start 168.75 37) (end 170.5 37) (width 0.84) (layer "B.Cu") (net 8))
 (segment (start 166.75 39) (end 167.75 38) (width 0.84) (layer "B.Cu") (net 8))
 (segment (start 178 37) (end 174.25 37) (width 0.84) (layer "B.Cu") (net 8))
 (segment (start 181 45.42) (end 181 40) (width 0.84) (layer "B.Cu") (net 8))
 (segment (start 166.25 41.625) (end 166.25 39) (width 0.84) (layer "B.Cu") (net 8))
 (segment (start 167.75 38) (end 168.75 37) (width 0.84) (layer "B.Cu") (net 8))
 (segment (start 178.545 45.42) (end 183.75 45.42) (width 0.84) (layer "B.Cu") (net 8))
 (segment (start 175.5 37) (end 174.25 37) (width 0.84) (layer "B.Cu") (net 8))
 (segment (start 166.25 39) (end 165.25 39) (width 0.84) (layer "B.Cu") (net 8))
 (segment (start 174.25 37) (end 173 37) (width 0.84) (layer "B.Cu") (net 8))
 (segment (start 165.25 39) (end 166.75 39) (width 0.84) (layer "B.Cu") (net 8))
 (segment (start 181 40) (end 178 37) (width 0.84) (layer "B.Cu") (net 8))
 (segment (start 133.975 57.025) (end 135.25 55.75) (width 0.84) (layer "B.Cu") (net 15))
 (segment (start 131 57.025) (end 133.975 57.025) (width 0.84) (layer "B.Cu") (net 15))
 (segment (start 147.225 54) (end 147.25 54.025) (width 0.84) (layer "B.Cu") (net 10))
 (segment (start 130.83 45.42) (end 132.95 45.42) (width 0.84) (layer "B.Cu") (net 10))
 (segment (start 128.75 47.5) (end 130.83 45.42) (width 0.84) (layer "B.Cu") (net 10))
 (segment (start 132.95 45.42) (end 139.13 45.42) (width 0.84) (layer "B.Cu") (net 10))
 (segment (start 127.4 36.05) (end 127 36.45) (width 0.84) (layer "B.Cu") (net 10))
 (segment (start 132.1 36.05) (end 127.4 36.05) (width 0.84) (layer "B.Cu") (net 10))
 (segment (start 131 54.485) (end 129.485 54.485) (width 0.84) (layer "B.Cu") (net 10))
 (segment (start 143.9 54) (end 143.9 46.65) (width 0.84) (layer "B.Cu") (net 10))
 (segment (start 132.95 36.9) (end 132.1 36.05) (width 0.84) (layer "B.Cu") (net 10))
 (segment (start 128.75 53.75) (end 128.75 47.5) (width 0.84) (layer "B.Cu") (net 10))
 (segment (start 143.9 46.65) (end 142.67 45.42) (width 0.84) (layer "B.Cu") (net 10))
 (segment (start 127 36.45) (end 127 38.5) (width 0.84) (layer "B.Cu") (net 10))
 (segment (start 132.95 45.42) (end 132.95 36.9) (width 0.84) (layer "B.Cu") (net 10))
 (segment (start 129.485 54.485) (end 128.75 53.75) (width 0.84) (layer "B.Cu") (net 10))
 (segment (start 143.9 54) (end 147.225 54) (width 0.84) (layer "B.Cu") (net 10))
 (segment (start 142.67 45.42) (end 139.13 45.42) (width 0.84) (layer "B.Cu") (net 10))
 (segment (start 181.46 47.96) (end 183.75 50.25) (width 0.84) (layer "B.Cu") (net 4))
 (segment (start 176.46 47.96) (end 178.545 47.96) (width 0.84) (layer "B.Cu") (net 4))
 (segment (start 170.5 39.25) (end 174 39.25) (width 0.84) (layer "B.Cu") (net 4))
 (segment (start 175.25 46.75) (end 176.46 47.96) (width 0.84) (layer "B.Cu") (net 4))
 (segment (start 175.25 40.5) (end 175.25 46.75) (width 0.84) (layer "B.Cu") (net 4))
 (segment (start 178.545 47.96) (end 181.46 47.96) (width 0.84) (layer "B.Cu") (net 4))
 (segment (start 174 39.25) (end 175.25 40.5) (width 0.84) (layer "B.Cu") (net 4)))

